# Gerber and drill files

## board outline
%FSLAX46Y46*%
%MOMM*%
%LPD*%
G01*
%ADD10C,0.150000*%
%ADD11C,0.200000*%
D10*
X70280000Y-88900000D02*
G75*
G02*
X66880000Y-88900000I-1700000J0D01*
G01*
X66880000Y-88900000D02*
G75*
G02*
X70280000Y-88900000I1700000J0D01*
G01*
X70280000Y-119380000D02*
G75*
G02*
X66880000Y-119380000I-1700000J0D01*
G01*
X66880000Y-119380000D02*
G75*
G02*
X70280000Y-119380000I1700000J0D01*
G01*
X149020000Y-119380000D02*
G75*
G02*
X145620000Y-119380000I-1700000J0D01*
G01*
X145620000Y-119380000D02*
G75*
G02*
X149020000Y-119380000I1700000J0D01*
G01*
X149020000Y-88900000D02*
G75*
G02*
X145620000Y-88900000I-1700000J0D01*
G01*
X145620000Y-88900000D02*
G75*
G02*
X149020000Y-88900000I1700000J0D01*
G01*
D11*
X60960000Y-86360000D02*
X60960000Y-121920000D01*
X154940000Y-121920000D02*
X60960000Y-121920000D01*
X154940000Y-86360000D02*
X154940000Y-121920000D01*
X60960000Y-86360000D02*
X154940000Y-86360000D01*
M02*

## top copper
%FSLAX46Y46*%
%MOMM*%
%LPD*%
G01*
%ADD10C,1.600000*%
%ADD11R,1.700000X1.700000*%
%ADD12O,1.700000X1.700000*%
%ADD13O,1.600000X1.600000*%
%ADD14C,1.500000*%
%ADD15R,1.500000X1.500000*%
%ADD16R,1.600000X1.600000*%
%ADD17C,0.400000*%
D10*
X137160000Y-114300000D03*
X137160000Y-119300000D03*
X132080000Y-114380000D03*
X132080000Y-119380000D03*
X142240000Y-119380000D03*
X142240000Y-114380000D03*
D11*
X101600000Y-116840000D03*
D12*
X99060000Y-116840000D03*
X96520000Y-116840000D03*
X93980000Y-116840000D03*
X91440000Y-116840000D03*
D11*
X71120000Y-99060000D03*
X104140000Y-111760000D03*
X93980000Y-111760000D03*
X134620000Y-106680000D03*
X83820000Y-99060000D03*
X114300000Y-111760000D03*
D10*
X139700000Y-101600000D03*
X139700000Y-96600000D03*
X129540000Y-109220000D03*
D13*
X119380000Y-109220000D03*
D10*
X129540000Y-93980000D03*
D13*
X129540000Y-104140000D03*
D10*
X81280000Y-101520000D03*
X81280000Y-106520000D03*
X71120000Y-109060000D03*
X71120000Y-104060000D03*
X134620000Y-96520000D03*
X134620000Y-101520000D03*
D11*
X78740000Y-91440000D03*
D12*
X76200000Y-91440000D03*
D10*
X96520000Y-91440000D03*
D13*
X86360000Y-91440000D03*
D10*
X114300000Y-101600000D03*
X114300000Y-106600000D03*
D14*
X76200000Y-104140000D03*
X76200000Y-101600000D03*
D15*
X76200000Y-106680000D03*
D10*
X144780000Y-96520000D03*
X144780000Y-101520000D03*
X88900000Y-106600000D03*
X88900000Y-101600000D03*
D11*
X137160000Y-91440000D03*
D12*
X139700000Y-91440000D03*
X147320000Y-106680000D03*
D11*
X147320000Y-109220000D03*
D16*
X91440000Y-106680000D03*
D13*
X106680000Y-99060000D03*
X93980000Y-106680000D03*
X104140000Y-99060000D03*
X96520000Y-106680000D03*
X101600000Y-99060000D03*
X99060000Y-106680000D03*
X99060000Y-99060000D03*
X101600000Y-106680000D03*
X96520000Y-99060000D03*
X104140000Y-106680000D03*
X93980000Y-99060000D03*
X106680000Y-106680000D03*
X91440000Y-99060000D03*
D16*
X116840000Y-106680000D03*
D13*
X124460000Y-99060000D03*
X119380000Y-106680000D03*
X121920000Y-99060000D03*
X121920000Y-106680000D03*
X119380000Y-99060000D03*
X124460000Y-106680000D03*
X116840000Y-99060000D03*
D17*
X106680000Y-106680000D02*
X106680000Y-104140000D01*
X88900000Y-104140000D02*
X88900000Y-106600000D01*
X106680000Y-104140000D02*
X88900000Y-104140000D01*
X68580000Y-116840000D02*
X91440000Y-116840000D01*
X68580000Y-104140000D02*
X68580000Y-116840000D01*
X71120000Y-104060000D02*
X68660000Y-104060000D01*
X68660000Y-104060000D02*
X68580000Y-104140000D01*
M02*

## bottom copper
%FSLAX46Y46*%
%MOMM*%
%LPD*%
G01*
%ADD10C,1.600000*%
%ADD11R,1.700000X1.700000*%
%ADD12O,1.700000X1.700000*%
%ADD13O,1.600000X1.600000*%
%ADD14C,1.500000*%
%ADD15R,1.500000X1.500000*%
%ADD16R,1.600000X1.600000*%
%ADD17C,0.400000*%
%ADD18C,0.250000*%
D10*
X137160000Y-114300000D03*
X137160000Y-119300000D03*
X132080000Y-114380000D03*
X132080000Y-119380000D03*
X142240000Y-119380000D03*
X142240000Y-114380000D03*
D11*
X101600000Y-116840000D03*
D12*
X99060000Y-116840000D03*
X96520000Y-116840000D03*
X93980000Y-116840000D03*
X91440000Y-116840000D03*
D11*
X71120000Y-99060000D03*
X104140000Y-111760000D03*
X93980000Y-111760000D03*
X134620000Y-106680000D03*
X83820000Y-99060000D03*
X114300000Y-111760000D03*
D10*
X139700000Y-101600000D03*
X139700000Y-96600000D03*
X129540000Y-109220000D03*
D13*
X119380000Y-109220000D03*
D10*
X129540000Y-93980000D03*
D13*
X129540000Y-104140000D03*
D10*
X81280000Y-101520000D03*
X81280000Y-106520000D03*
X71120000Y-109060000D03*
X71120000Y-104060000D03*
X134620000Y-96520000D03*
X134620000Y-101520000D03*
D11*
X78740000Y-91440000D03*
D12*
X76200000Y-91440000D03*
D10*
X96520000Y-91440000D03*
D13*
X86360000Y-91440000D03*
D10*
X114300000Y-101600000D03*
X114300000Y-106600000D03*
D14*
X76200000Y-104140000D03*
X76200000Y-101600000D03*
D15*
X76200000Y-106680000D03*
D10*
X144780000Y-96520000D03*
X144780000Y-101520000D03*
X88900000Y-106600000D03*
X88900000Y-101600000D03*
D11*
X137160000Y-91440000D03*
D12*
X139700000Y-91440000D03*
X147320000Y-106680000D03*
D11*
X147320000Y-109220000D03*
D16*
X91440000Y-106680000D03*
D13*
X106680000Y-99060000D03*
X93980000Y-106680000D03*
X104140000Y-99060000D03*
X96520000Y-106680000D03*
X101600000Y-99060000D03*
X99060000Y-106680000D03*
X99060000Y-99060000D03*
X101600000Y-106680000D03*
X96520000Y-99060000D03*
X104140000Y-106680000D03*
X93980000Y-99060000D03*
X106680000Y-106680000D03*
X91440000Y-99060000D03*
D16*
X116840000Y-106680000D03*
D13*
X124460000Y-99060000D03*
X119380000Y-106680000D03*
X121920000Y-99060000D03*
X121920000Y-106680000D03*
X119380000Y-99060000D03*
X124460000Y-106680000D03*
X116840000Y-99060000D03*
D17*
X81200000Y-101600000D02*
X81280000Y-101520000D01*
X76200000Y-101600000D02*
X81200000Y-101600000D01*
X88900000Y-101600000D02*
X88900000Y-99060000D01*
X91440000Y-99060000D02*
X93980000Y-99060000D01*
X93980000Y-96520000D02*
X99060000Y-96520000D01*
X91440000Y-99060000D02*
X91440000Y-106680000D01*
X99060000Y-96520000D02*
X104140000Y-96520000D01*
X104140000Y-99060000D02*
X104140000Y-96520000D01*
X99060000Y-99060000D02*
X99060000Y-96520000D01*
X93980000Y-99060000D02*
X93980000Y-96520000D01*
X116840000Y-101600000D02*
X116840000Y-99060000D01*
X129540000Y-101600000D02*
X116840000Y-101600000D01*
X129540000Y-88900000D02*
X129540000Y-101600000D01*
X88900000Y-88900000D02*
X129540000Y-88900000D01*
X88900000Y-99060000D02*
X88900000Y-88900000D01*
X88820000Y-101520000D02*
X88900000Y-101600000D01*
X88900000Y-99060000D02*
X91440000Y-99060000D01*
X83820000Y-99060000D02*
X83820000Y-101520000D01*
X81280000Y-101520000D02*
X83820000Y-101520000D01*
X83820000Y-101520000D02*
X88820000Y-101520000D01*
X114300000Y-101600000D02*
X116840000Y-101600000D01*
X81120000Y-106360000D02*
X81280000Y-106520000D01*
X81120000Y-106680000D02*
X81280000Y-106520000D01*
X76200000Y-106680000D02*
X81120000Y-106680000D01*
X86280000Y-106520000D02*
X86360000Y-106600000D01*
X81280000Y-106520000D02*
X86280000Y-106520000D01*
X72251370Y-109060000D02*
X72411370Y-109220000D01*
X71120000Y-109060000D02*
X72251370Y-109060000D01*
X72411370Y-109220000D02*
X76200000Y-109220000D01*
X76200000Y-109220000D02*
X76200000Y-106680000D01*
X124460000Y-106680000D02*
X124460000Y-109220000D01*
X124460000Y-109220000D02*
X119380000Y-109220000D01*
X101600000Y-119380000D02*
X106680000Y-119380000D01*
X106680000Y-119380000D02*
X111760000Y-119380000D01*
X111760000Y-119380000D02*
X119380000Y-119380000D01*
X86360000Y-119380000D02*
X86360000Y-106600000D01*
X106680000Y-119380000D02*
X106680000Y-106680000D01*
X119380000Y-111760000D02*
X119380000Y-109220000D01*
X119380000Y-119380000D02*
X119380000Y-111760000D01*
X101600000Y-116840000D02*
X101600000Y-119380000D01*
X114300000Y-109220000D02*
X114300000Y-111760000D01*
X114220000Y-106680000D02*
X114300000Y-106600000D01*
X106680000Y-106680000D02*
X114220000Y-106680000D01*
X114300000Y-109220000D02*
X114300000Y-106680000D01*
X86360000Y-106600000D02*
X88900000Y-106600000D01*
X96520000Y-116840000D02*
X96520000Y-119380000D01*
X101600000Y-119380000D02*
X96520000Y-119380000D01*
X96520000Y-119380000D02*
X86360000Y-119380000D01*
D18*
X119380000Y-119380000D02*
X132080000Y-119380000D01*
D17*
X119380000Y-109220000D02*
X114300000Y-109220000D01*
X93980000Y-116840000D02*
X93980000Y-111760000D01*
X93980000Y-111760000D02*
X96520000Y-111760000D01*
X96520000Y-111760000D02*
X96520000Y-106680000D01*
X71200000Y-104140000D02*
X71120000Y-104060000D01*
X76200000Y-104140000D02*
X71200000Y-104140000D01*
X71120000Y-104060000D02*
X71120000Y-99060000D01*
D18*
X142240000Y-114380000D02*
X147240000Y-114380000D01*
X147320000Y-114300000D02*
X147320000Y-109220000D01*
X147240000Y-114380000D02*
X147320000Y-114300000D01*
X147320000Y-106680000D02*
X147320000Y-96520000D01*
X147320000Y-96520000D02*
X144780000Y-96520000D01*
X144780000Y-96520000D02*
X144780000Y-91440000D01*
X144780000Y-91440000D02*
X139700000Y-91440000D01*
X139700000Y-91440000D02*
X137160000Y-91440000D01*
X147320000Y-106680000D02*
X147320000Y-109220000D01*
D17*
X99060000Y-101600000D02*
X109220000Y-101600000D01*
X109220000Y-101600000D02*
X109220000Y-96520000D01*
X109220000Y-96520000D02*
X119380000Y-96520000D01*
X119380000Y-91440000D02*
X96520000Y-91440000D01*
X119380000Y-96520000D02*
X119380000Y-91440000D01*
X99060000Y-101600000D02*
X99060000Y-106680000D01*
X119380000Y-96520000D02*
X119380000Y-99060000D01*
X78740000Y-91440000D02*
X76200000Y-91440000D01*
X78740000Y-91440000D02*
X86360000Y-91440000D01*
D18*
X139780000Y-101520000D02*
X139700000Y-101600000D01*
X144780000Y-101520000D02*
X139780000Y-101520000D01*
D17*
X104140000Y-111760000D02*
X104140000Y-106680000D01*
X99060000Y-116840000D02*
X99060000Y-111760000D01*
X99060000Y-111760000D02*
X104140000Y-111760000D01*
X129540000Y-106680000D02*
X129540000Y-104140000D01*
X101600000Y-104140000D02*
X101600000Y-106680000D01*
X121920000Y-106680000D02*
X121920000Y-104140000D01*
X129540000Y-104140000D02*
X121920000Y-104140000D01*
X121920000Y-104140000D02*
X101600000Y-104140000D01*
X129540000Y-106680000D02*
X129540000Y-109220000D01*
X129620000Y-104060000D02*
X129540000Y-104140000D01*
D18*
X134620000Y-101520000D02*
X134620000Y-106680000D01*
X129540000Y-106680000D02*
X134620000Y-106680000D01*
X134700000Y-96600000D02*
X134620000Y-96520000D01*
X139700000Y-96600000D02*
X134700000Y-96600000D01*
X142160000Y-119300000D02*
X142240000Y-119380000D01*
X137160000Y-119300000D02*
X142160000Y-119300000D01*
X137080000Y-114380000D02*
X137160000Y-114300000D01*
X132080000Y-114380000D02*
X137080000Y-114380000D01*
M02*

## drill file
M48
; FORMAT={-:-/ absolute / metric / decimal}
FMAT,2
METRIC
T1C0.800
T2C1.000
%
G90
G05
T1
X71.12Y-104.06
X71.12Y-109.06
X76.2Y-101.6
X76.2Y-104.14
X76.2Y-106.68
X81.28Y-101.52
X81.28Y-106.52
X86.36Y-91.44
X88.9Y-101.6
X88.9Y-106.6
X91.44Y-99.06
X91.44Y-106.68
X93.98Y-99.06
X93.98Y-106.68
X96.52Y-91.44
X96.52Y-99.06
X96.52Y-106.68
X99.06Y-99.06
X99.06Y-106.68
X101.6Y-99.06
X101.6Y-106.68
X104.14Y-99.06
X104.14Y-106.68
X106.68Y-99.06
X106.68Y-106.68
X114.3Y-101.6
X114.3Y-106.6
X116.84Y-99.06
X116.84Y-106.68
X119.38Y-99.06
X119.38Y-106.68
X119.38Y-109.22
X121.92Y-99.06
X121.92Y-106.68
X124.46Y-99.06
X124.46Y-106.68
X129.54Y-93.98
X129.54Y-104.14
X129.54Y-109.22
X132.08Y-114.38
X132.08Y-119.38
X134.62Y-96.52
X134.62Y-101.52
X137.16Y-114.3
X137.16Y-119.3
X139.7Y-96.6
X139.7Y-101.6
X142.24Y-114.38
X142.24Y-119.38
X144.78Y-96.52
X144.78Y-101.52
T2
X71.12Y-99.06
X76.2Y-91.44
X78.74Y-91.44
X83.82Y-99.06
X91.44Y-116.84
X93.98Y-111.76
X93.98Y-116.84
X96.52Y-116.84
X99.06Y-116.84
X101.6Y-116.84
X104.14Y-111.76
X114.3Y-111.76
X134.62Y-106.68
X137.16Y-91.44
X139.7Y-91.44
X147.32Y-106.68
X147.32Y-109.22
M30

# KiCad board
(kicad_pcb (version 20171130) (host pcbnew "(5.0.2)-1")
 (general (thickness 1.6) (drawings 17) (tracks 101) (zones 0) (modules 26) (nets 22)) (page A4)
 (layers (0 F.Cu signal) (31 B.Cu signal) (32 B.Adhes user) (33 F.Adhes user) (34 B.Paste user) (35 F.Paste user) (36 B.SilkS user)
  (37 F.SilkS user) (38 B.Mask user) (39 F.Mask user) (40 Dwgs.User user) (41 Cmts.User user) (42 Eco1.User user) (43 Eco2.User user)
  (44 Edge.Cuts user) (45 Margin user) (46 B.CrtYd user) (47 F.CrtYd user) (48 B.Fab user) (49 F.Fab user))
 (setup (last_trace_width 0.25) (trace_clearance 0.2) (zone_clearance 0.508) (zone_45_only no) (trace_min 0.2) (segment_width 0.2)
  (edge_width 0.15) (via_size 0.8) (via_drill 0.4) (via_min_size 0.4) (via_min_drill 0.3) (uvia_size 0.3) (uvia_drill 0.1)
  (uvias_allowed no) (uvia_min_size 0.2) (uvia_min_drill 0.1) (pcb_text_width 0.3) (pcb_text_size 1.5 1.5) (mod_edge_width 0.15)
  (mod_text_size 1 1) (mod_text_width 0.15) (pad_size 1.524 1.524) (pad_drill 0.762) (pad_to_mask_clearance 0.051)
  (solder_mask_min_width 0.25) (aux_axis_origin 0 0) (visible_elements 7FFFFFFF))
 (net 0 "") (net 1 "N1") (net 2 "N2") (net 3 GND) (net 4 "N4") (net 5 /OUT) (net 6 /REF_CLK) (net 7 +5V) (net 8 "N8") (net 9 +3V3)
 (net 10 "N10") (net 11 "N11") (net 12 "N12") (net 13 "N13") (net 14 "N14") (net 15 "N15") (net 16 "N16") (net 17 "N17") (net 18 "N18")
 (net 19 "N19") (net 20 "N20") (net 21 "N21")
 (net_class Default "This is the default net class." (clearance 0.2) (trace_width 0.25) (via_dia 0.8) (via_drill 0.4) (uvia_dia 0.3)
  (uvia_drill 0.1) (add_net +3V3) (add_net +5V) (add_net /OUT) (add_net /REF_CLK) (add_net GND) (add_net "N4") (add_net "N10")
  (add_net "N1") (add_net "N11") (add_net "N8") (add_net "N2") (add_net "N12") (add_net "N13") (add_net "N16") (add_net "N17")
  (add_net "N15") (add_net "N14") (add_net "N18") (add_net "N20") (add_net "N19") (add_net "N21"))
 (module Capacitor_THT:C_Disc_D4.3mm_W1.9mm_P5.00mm (layer F.Cu) (at 137.16 114.3 270)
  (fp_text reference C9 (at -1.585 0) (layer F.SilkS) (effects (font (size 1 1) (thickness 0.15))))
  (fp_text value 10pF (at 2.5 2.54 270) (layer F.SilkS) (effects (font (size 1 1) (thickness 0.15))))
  (pad 1 thru_hole circle (at 0 0 270) (size 1.6 1.6) (drill 0.8) (layers *.Cu *.Mask) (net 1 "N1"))
  (pad 2 thru_hole circle (at 5 0 270) (size 1.6 1.6) (drill 0.8) (layers *.Cu *.Mask) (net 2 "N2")))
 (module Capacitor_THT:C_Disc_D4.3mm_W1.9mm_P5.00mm (layer F.Cu) (at 132.08 119.38 90)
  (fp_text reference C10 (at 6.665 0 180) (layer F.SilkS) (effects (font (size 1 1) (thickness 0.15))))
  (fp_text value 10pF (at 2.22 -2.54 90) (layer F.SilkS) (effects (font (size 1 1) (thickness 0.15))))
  (pad 2 thru_hole circle (at 5 0 90) (size 1.6 1.6) (drill 0.8) (layers *.Cu *.Mask) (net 1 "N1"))
  (pad 1 thru_hole circle (at 0 0 90) (size 1.6 1.6) (drill 0.8) (layers *.Cu *.Mask) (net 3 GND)))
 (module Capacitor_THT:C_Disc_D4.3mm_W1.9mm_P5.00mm (layer F.Cu) (at 142.24 119.38 90)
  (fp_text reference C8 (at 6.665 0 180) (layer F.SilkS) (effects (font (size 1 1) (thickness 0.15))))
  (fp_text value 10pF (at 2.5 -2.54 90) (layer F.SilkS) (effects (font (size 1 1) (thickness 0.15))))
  (pad 1 thru_hole circle (at 0 0 90) (size 1.6 1.6) (drill 0.8) (layers *.Cu *.Mask) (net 2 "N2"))
  (pad 2 thru_hole circle (at 5 0 90) (size 1.6 1.6) (drill 0.8) (layers *.Cu *.Mask) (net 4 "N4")))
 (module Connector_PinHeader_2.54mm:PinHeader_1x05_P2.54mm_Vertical (layer F.Cu) (at 101.6 116.84 270)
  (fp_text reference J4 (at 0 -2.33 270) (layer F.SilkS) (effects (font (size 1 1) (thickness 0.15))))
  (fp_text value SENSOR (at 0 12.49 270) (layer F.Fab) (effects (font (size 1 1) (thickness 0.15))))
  (pad 1 thru_hole rect (at 0 0 270) (size 1.7 1.7) (drill 1) (layers *.Cu *.Mask) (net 3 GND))
  (pad 2 thru_hole oval (at 0 2.54 270) (size 1.7 1.7) (drill 1) (layers *.Cu *.Mask) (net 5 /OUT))
  (pad 3 thru_hole oval (at 0 5.08 270) (size 1.7 1.7) (drill 1) (layers *.Cu *.Mask) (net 3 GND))
  (pad 4 thru_hole oval (at 0 7.62 270) (size 1.7 1.7) (drill 1) (layers *.Cu *.Mask) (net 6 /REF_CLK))
  (pad 5 thru_hole oval (at 0 10.16 270) (size 1.7 1.7) (drill 1) (layers *.Cu *.Mask) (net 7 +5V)))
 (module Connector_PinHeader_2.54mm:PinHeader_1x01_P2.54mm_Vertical (layer F.Cu) (at 71.12 99.06)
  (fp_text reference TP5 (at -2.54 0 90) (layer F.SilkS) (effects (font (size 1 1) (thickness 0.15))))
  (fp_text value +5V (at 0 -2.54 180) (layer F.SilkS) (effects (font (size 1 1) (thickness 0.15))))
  (pad 1 thru_hole rect (at 0 0) (size 1.7 1.7) (drill 1) (layers *.Cu *.Mask) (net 7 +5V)))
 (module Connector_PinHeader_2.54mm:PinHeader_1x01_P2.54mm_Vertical (layer F.Cu) (at 104.14 111.76)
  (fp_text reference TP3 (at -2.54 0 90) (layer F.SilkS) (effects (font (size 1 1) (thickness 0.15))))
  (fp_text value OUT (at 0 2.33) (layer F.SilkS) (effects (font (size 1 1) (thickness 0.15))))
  (pad 1 thru_hole rect (at 0 0) (size 1.7 1.7) (drill 1) (layers *.Cu *.Mask) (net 5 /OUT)))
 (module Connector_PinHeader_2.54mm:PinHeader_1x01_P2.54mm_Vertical (layer F.Cu) (at 93.98 111.76)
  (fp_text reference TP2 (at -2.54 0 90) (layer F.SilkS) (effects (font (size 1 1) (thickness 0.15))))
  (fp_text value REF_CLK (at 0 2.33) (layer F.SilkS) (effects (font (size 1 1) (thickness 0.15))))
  (pad 1 thru_hole rect (at 0 0) (size 1.7 1.7) (drill 1) (layers *.Cu *.Mask) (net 6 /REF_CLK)))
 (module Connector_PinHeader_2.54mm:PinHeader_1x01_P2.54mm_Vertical (layer F.Cu) (at 134.62 106.68)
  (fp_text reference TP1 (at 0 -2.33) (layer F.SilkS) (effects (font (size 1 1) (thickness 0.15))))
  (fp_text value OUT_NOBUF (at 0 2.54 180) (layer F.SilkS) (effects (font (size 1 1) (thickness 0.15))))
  (pad 1 thru_hole rect (at 0 0) (size 1.7 1.7) (drill 1) (layers *.Cu *.Mask) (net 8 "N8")))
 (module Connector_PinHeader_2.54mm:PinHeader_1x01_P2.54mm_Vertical (layer F.Cu) (at 83.82 99.06)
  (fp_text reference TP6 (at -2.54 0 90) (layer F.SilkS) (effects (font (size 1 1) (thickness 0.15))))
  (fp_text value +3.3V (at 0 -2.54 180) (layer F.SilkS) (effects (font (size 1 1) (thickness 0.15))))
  (pad 1 thru_hole rect (at 0 0) (size 1.7 1.7) (drill 1) (layers *.Cu *.Mask) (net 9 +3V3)))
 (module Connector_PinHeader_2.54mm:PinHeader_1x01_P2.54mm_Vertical (layer F.Cu) (at 114.3 111.76)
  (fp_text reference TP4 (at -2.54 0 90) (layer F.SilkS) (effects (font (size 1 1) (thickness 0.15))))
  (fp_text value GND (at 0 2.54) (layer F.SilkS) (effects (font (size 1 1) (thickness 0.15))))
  (pad 1 thru_hole rect (at 0 0) (size 1.7 1.7) (drill 1) (layers *.Cu *.Mask) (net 3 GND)))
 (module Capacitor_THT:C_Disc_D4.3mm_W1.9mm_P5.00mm (layer F.Cu) (at 139.7 101.6 90)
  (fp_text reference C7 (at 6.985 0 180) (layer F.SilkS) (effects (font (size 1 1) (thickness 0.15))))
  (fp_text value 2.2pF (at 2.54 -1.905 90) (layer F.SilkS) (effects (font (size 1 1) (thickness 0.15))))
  (pad 1 thru_hole circle (at 0 0 90) (size 1.6 1.6) (drill 0.8) (layers *.Cu *.Mask) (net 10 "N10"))
  (pad 2 thru_hole circle (at 5 0 90) (size 1.6 1.6) (drill 0.8) (layers *.Cu *.Mask) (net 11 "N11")))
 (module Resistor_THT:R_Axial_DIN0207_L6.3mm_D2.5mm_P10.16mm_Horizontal (layer F.Cu) (at 129.54 109.22 180)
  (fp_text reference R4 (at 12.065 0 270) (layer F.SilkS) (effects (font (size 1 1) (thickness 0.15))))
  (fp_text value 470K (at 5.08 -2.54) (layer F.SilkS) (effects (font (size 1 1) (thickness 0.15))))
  (pad 1 thru_hole circle (at 0 0 180) (size 1.6 1.6) (drill 0.8) (layers *.Cu *.Mask) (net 8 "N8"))
  (pad 2 thru_hole oval (at 10.16 0 180) (size 1.6 1.6) (drill 0.8) (layers *.Cu *.Mask) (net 3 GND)))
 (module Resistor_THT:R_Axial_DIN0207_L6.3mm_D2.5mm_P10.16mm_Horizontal (layer F.Cu) (at 129.54 93.98 270)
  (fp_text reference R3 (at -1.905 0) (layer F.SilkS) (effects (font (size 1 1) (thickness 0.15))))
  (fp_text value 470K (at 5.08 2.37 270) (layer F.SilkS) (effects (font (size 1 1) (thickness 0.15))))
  (pad 1 thru_hole circle (at 0 0 270) (size 1.6 1.6) (drill 0.8) (layers *.Cu *.Mask) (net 9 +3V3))
  (pad 2 thru_hole oval (at 10.16 0 270) (size 1.6 1.6) (drill 0.8) (layers *.Cu *.Mask) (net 8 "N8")))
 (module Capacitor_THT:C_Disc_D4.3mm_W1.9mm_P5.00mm (layer F.Cu) (at 81.28 101.52 270)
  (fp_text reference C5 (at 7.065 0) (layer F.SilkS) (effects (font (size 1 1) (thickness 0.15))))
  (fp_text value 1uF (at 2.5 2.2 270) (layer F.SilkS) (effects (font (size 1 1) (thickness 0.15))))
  (pad 1 thru_hole circle (at 0 0 270) (size 1.6 1.6) (drill 0.8) (layers *.Cu *.Mask) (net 9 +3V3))
  (pad 2 thru_hole circle (at 5 0 270) (size 1.6 1.6) (drill 0.8) (layers *.Cu *.Mask) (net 3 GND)))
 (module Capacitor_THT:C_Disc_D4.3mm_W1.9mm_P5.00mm (layer F.Cu) (at 71.12 104.06 270)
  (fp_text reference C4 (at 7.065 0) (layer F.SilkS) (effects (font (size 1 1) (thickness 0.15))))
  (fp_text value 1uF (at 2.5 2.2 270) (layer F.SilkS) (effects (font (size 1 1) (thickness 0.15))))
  (pad 2 thru_hole circle (at 5 0 270) (size 1.6 1.6) (drill 0.8) (layers *.Cu *.Mask) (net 3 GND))
  (pad 1 thru_hole circle (at 0 0 270) (size 1.6 1.6) (drill 0.8) (layers *.Cu *.Mask) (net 7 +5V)))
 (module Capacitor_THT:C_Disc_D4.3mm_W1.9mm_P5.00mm (layer F.Cu) (at 134.62 96.52 270)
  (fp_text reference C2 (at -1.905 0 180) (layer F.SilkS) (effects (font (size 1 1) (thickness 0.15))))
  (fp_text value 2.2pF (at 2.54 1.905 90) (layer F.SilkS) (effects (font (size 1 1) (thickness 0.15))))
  (pad 1 thru_hole circle (at 0 0 270) (size 1.6 1.6) (drill 0.8) (layers *.Cu *.Mask) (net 11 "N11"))
  (pad 2 thru_hole circle (at 5 0 270) (size 1.6 1.6) (drill 0.8) (layers *.Cu *.Mask) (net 8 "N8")))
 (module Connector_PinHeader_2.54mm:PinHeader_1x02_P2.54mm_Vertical (layer F.Cu) (at 78.74 91.44 270)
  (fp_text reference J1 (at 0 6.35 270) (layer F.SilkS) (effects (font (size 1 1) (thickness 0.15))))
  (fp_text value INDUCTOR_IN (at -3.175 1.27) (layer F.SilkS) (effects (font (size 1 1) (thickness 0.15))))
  (pad 1 thru_hole rect (at 0 0 270) (size 1.7 1.7) (drill 1) (layers *.Cu *.Mask) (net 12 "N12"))
  (pad 2 thru_hole oval (at 0 2.54 270) (size 1.7 1.7) (drill 1) (layers *.Cu *.Mask) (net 12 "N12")))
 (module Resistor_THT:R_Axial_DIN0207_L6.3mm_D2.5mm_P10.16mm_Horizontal (layer F.Cu) (at 96.52 91.44 180)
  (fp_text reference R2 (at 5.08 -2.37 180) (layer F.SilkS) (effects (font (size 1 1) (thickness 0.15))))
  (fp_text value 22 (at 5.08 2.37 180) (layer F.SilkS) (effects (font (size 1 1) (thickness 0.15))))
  (pad 1 thru_hole circle (at 0 0 180) (size 1.6 1.6) (drill 0.8) (layers *.Cu *.Mask) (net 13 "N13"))
  (pad 2 thru_hole oval (at 10.16 0 180) (size 1.6 1.6) (drill 0.8) (layers *.Cu *.Mask) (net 12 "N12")))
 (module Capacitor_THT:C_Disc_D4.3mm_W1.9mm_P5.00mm (layer F.Cu) (at 114.3 101.6 270)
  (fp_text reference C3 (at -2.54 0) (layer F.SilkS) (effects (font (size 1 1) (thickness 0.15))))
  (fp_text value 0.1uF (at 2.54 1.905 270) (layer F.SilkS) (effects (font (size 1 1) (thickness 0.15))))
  (pad 1 thru_hole circle (at 0 0 270) (size 1.6 1.6) (drill 0.8) (layers *.Cu *.Mask) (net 9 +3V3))
  (pad 2 thru_hole circle (at 5 0 270) (size 1.6 1.6) (drill 0.8) (layers *.Cu *.Mask) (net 3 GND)))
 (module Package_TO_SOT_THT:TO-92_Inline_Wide (layer F.Cu) (at 76.2 106.68 90)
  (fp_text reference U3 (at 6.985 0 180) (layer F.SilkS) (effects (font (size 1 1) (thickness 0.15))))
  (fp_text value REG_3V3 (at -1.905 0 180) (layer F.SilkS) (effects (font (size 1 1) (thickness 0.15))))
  (pad 2 thru_hole circle (at 2.54 0 180) (size 1.5 1.5) (drill 0.8) (layers *.Cu *.Mask) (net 7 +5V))
  (pad 3 thru_hole circle (at 5.08 0 180) (size 1.5 1.5) (drill 0.8) (layers *.Cu *.Mask) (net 9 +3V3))
  (pad 1 thru_hole rect (at 0 0 180) (size 1.5 1.5) (drill 0.8) (layers *.Cu *.Mask) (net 3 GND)))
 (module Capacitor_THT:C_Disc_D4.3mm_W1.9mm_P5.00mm (layer F.Cu) (at 144.78 96.52 270)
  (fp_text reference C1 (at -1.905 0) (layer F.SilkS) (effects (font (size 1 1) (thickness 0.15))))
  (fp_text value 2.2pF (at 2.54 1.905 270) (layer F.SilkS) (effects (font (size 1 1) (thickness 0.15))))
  (pad 1 thru_hole circle (at 0 0 270) (size 1.6 1.6) (drill 0.8) (layers *.Cu *.Mask) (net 4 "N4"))
  (pad 2 thru_hole circle (at 5 0 270) (size 1.6 1.6) (drill 0.8) (layers *.Cu *.Mask) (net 10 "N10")))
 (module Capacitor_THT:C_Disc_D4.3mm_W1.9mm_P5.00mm (layer F.Cu) (at 88.9 101.6 270)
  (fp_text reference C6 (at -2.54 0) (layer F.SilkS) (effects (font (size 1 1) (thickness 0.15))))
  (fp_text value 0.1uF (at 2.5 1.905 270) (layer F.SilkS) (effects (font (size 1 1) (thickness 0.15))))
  (pad 2 thru_hole circle (at 5 0 270) (size 1.6 1.6) (drill 0.8) (layers *.Cu *.Mask) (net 3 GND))
  (pad 1 thru_hole circle (at 0 0 270) (size 1.6 1.6) (drill 0.8) (layers *.Cu *.Mask) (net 9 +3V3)))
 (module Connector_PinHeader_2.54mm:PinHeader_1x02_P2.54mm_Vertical (layer F.Cu) (at 137.16 91.44 90)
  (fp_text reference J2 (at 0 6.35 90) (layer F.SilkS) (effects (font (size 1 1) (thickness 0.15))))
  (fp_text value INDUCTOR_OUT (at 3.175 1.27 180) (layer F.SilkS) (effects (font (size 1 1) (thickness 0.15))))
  (pad 1 thru_hole rect (at 0 0 90) (size 1.7 1.7) (drill 1) (layers *.Cu *.Mask) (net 4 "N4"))
  (pad 2 thru_hole oval (at 0 2.54 90) (size 1.7 1.7) (drill 1) (layers *.Cu *.Mask) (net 4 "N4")))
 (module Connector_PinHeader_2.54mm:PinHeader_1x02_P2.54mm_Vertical (layer F.Cu) (at 147.32 109.22 180)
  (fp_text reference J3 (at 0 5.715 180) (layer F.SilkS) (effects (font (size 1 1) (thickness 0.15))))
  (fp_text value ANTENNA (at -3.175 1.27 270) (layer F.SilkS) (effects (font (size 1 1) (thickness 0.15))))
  (pad 2 thru_hole oval (at 0 2.54 180) (size 1.7 1.7) (drill 1) (layers *.Cu *.Mask) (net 4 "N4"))
  (pad 1 thru_hole rect (at 0 0 180) (size 1.7 1.7) (drill 1) (layers *.Cu *.Mask) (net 4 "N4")))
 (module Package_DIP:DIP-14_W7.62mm (layer F.Cu) (at 91.44 106.68 90)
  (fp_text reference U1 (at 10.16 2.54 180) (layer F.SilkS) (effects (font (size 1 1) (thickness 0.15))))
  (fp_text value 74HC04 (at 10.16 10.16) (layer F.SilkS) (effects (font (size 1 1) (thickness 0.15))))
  (pad 1 thru_hole rect (at 0 0 90) (size 1.6 1.6) (drill 0.8) (layers *.Cu *.Mask) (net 9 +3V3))
  (pad 8 thru_hole oval (at 7.62 15.24 90) (size 1.6 1.6) (drill 0.8) (layers *.Cu *.Mask) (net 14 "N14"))
  (pad 2 thru_hole oval (at 0 2.54 90) (size 1.6 1.6) (drill 0.8) (layers *.Cu *.Mask) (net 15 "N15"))
  (pad 9 thru_hole oval (at 7.62 12.7 90) (size 1.6 1.6) (drill 0.8) (layers *.Cu *.Mask) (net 9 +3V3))
  (pad 3 thru_hole oval (at 0 5.08 90) (size 1.6 1.6) (drill 0.8) (layers *.Cu *.Mask) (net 6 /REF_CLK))
  (pad 10 thru_hole oval (at 7.62 10.16 90) (size 1.6 1.6) (drill 0.8) (layers *.Cu *.Mask) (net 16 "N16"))
  (pad 4 thru_hole oval (at 0 7.62 90) (size 1.6 1.6) (drill 0.8) (layers *.Cu *.Mask) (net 13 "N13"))
  (pad 11 thru_hole oval (at 7.62 7.62 90) (size 1.6 1.6) (drill 0.8) (layers *.Cu *.Mask) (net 9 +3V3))
  (pad 5 thru_hole oval (at 0 10.16 90) (size 1.6 1.6) (drill 0.8) (layers *.Cu *.Mask) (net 8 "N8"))
  (pad 12 thru_hole oval (at 7.62 5.08 90) (size 1.6 1.6) (drill 0.8) (layers *.Cu *.Mask) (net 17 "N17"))
  (pad 6 thru_hole oval (at 0 12.7 90) (size 1.6 1.6) (drill 0.8) (layers *.Cu *.Mask) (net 5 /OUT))
  (pad 13 thru_hole oval (at 7.62 2.54 90) (size 1.6 1.6) (drill 0.8) (layers *.Cu *.Mask) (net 9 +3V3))
  (pad 7 thru_hole oval (at 0 15.24 90) (size 1.6 1.6) (drill 0.8) (layers *.Cu *.Mask) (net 3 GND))
  (pad 14 thru_hole oval (at 7.62 0 90) (size 1.6 1.6) (drill 0.8) (layers *.Cu *.Mask) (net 9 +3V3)))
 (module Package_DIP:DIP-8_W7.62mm (layer F.Cu) (at 116.84 106.68 90)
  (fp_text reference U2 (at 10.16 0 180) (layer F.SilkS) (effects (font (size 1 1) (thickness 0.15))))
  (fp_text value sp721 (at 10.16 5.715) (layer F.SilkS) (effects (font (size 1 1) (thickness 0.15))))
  (pad 1 thru_hole rect (at 0 0 90) (size 1.6 1.6) (drill 0.8) (layers *.Cu *.Mask) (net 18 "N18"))
  (pad 5 thru_hole oval (at 7.62 7.62 90) (size 1.6 1.6) (drill 0.8) (layers *.Cu *.Mask) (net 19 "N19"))
  (pad 2 thru_hole oval (at 0 2.54 90) (size 1.6 1.6) (drill 0.8) (layers *.Cu *.Mask) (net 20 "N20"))
  (pad 6 thru_hole oval (at 7.62 5.08 90) (size 1.6 1.6) (drill 0.8) (layers *.Cu *.Mask) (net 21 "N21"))
  (pad 3 thru_hole oval (at 0 5.08 90) (size 1.6 1.6) (drill 0.8) (layers *.Cu *.Mask) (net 8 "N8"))
  (pad 7 thru_hole oval (at 7.62 2.54 90) (size 1.6 1.6) (drill 0.8) (layers *.Cu *.Mask) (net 13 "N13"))
  (pad 4 thru_hole oval (at 0 7.62 90) (size 1.6 1.6) (drill 0.8) (layers *.Cu *.Mask) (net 3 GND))
  (pad 8 thru_hole oval (at 7.62 0 90) (size 1.6 1.6) (drill 0.8) (layers *.Cu *.Mask) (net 9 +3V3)))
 (gr_circle (center 68.58 88.9) (end 70.28 88.9) (layer Edge.Cuts) (width 0.15))
 (gr_circle (center 68.58 119.38) (end 70.28 119.38) (layer Edge.Cuts) (width 0.15))
 (gr_circle (center 147.32 119.38) (end 149.02 119.38) (layer Edge.Cuts) (width 0.15))
 (gr_circle (center 147.32 88.9) (end 149.02 88.9) (layer Edge.Cuts) (width 0.15))
 (gr_line (start 60.96 86.36) (end 60.96 121.92) (layer Edge.Cuts) (width 0.2))
 (gr_line (start 154.94 121.92) (end 60.96 121.92) (layer Edge.Cuts) (width 0.2))
 (gr_line (start 154.94 86.36) (end 154.94 121.92) (layer Edge.Cuts) (width 0.2))
 (gr_line (start 60.96 86.36) (end 154.94 86.36) (layer Edge.Cuts) (width 0.2))
 (segment (start 81.2 101.6) (end 81.28 101.52) (width 0.4) (layer B.Cu) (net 9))
 (segment (start 76.2 101.6) (end 81.2 101.6) (width 0.4) (layer B.Cu) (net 9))
 (segment (start 88.9 101.6) (end 88.9 99.06) (width 0.4) (layer B.Cu) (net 9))
 (segment (start 91.44 99.06) (end 93.98 99.06) (width 0.4) (layer B.Cu) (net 9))
 (segment (start 93.98 96.52) (end 99.06 96.52) (width 0.4) (layer B.Cu) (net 9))
 (segment (start 91.44 99.06) (end 91.44 106.68) (width 0.4) (layer B.Cu) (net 9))
 (segment (start 99.06 96.52) (end 104.14 96.52) (width 0.4) (layer B.Cu) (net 9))
 (segment (start 104.14 99.06) (end 104.14 96.52) (width 0.4) (layer B.Cu) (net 9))
 (segment (start 99.06 99.06) (end 99.06 96.52) (width 0.4) (layer B.Cu) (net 9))
 (segment (start 93.98 99.06) (end 93.98 96.52) (width 0.4) (layer B.Cu) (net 9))
 (segment (start 116.84 101.6) (end 116.84 99.06) (width 0.4) (layer B.Cu) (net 9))
 (segment (start 129.54 101.6) (end 116.84 101.6) (width 0.4) (layer B.Cu) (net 9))
 (segment (start 129.54 88.9) (end 129.54 101.6) (width 0.4) (layer B.Cu) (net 9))
 (segment (start 88.9 88.9) (end 129.54 88.9) (width 0.4) (layer B.Cu) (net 9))
 (segment (start 88.9 99.06) (end 88.9 88.9) (width 0.4) (layer B.Cu) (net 9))
 (segment (start 88.82 101.52) (end 88.9 101.6) (width 0.4) (layer B.Cu) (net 9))
 (segment (start 88.9 99.06) (end 91.44 99.06) (width 0.4) (layer B.Cu) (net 9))
 (segment (start 83.82 99.06) (end 83.82 101.52) (width 0.4) (layer B.Cu) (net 9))
 (segment (start 81.28 101.52) (end 83.82 101.52) (width 0.4) (layer B.Cu) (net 9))
 (segment (start 83.82 101.52) (end 88.82 101.52) (width 0.4) (layer B.Cu) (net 9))
 (segment (start 114.3 101.6) (end 116.84 101.6) (width 0.4) (layer B.Cu) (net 9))
 (segment (start 81.12 106.36) (end 81.28 106.52) (width 0.4) (layer B.Cu) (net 3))
 (segment (start 81.12 106.68) (end 81.28 106.52) (width 0.4) (layer B.Cu) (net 3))
 (segment (start 76.2 106.68) (end 81.12 106.68) (width 0.4) (layer B.Cu) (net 3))
 (segment (start 86.28 106.52) (end 86.36 106.6) (width 0.4) (layer B.Cu) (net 3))
 (segment (start 81.28 106.52) (end 86.28 106.52) (width 0.4) (layer B.Cu) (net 3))
 (segment (start 72.25137 109.06) (end 72.41137 109.22) (width 0.4) (layer B.Cu) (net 3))
 (segment (start 71.12 109.06) (end 72.25137 109.06) (width 0.4) (layer B.Cu) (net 3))
 (segment (start 72.41137 109.22) (end 76.2 109.22) (width 0.4) (layer B.Cu) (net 3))
 (segment (start 76.2 109.22) (end 76.2 106.68) (width 0.4) (layer B.Cu) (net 3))
 (segment (start 124.46 106.68) (end 124.46 109.22) (width 0.4) (layer B.Cu) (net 3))
 (segment (start 124.46 109.22) (end 119.38 109.22) (width 0.4) (layer B.Cu) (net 3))
 (segment (start 101.6 119.38) (end 106.68 119.38) (width 0.4) (layer B.Cu) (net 3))
 (segment (start 106.68 119.38) (end 111.76 119.38) (width 0.4) (layer B.Cu) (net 3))
 (segment (start 111.76 119.38) (end 119.38 119.38) (width 0.4) (layer B.Cu) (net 3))
 (segment (start 86.36 119.38) (end 86.36 106.6) (width 0.4) (layer B.Cu) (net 3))
 (segment (start 106.68 119.38) (end 106.68 106.68) (width 0.4) (layer B.Cu) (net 3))
 (segment (start 119.38 111.76) (end 119.38 109.22) (width 0.4) (layer B.Cu) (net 3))
 (segment (start 119.38 119.38) (end 119.38 111.76) (width 0.4) (layer B.Cu) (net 3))
 (segment (start 101.6 116.84) (end 101.6 119.38) (width 0.4) (layer B.Cu) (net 3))
 (segment (start 114.3 109.22) (end 114.3 111.76) (width 0.4) (layer B.Cu) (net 3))
 (segment (start 106.68 106.68) (end 106.68 104.14) (width 0.4) (layer F.Cu) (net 3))
 (segment (start 114.22 106.68) (end 114.3 106.6) (width 0.4) (layer B.Cu) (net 3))
 (segment (start 106.68 106.68) (end 114.22 106.68) (width 0.4) (layer B.Cu) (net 3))
 (segment (start 114.3 109.22) (end 114.3 106.68) (width 0.4) (layer B.Cu) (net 3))
 (segment (start 86.36 106.6) (end 88.9 106.6) (width 0.4) (layer B.Cu) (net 3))
 (segment (start 88.9 104.14) (end 88.9 106.6) (width 0.4) (layer F.Cu) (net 3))
 (segment (start 106.68 104.14) (end 88.9 104.14) (width 0.4) (layer F.Cu) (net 3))
 (segment (start 96.52 116.84) (end 96.52 119.38) (width 0.4) (layer B.Cu) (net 3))
 (segment (start 101.6 119.38) (end 96.52 119.38) (width 0.4) (layer B.Cu) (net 3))
 (segment (start 96.52 119.38) (end 86.36 119.38) (width 0.4) (layer B.Cu) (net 3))
 (segment (start 119.38 119.38) (end 132.08 119.38) (width 0.25) (layer B.Cu) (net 3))
 (segment (start 119.38 109.22) (end 114.3 109.22) (width 0.4) (layer B.Cu) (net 3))
 (segment (start 93.98 116.84) (end 93.98 111.76) (width 0.4) (layer B.Cu) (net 6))
 (segment (start 93.98 111.76) (end 96.52 111.76) (width 0.4) (layer B.Cu) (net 6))
 (segment (start 96.52 111.76) (end 96.52 106.68) (width 0.4) (layer B.Cu) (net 6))
 (segment (start 71.2 104.14) (end 71.12 104.06) (width 0.4) (layer B.Cu) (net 7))
 (segment (start 76.2 104.14) (end 71.2 104.14) (width 0.4) (layer B.Cu) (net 7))
 (segment (start 71.12 104.06) (end 71.12 99.06) (width 0.4) (layer B.Cu) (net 7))
 (segment (start 68.58 116.84) (end 91.44 116.84) (width 0.4) (layer F.Cu) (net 7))
 (segment (start 68.58 104.14) (end 68.58 116.84) (width 0.4) (layer F.Cu) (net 7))
 (segment (start 71.12 104.06) (end 68.66 104.06) (width 0.4) (layer F.Cu) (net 7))
 (segment (start 68.66 104.06) (end 68.58 104.14) (width 0.4) (layer F.Cu) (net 7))
 (segment (start 142.24 114.38) (end 147.24 114.38) (width 0.25) (layer B.Cu) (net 4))
 (segment (start 147.32 114.3) (end 147.32 109.22) (width 0.25) (layer B.Cu) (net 4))
 (segment (start 147.24 114.38) (end 147.32 114.3) (width 0.25) (layer B.Cu) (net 4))
 (segment (start 147.32 106.68) (end 147.32 96.52) (width 0.25) (layer B.Cu) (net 4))
 (segment (start 147.32 96.52) (end 144.78 96.52) (width 0.25) (layer B.Cu) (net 4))
 (segment (start 144.78 96.52) (end 144.78 91.44) (width 0.25) (layer B.Cu) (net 4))
 (segment (start 144.78 91.44) (end 139.7 91.44) (width 0.25) (layer B.Cu) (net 4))
 (segment (start 139.7 91.44) (end 137.16 91.44) (width 0.25) (layer B.Cu) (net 4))
 (segment (start 147.32 106.68) (end 147.32 109.22) (width 0.25) (layer B.Cu) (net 4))
 (segment (start 99.06 101.6) (end 109.22 101.6) (width 0.4) (layer B.Cu) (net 13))
 (segment (start 109.22 101.6) (end 109.22 96.52) (width 0.4) (layer B.Cu) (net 13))
 (segment (start 109.22 96.52) (end 119.38 96.52) (width 0.4) (layer B.Cu) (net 13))
 (segment (start 119.38 91.44) (end 96.52 91.44) (width 0.4) (layer B.Cu) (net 13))
 (segment (start 119.38 96.52) (end 119.38 91.44) (width 0.4) (layer B.Cu) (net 13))
 (segment (start 99.06 101.6) (end 99.06 106.68) (width 0.4) (layer B.Cu) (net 13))
 (segment (start 119.38 96.52) (end 119.38 99.06) (width 0.4) (layer B.Cu) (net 13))
 (segment (start 78.74 91.44) (end 76.2 91.44) (width 0.4) (layer B.Cu) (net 12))
 (segment (start 78.74 91.44) (end 86.36 91.44) (width 0.4) (layer B.Cu) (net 12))
 (segment (start 139.78 101.52) (end 139.7 101.6) (width 0.25) (layer B.Cu) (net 10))
 (segment (start 144.78 101.52) (end 139.78 101.52) (width 0.25) (layer B.Cu) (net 10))
 (segment (start 104.14 111.76) (end 104.14 106.68) (width 0.4) (layer B.Cu) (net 5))
 (segment (start 99.06 116.84) (end 99.06 111.76) (width 0.4) (layer B.Cu) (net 5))
 (segment (start 99.06 111.76) (end 104.14 111.76) (width 0.4) (layer B.Cu) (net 5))
 (segment (start 129.54 106.68) (end 129.54 104.14) (width 0.4) (layer B.Cu) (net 8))
 (segment (start 101.6 104.14) (end 101.6 106.68) (width 0.4) (layer B.Cu) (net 8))
 (segment (start 121.92 106.68) (end 121.92 104.14) (width 0.4) (layer B.Cu) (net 8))
 (segment (start 129.54 104.14) (end 121.92 104.14) (width 0.4) (layer B.Cu) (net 8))
 (segment (start 121.92 104.14) (end 101.6 104.14) (width 0.4) (layer B.Cu) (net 8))
 (segment (start 129.54 106.68) (end 129.54 109.22) (width 0.4) (layer B.Cu) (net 8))
 (segment (start 129.62 104.06) (end 129.54 104.14) (width 0.4) (layer B.Cu) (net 8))
 (segment (start 134.62 101.52) (end 134.62 106.68) (width 0.25) (layer B.Cu) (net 8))
 (segment (start 129.54 106.68) (end 134.62 106.68) (width 0.25) (layer B.Cu) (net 8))
 (segment (start 134.7 96.6) (end 134.62 96.52) (width 0.25) (layer B.Cu) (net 11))
 (segment (start 139.7 96.6) (end 134.7 96.6) (width 0.25) (layer B.Cu) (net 11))
 (segment (start 142.16 119.3) (end 142.24 119.38) (width 0.25) (layer B.Cu) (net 2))
 (segment (start 137.16 119.3) (end 142.16 119.3) (width 0.25) (layer B.Cu) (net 2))
 (segment (start 137.08 114.38) (end 137.16 114.3) (width 0.25) (layer B.Cu) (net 1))
 (segment (start 132.08 114.38) (end 137.08 114.38) (width 0.25) (layer B.Cu) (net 1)))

